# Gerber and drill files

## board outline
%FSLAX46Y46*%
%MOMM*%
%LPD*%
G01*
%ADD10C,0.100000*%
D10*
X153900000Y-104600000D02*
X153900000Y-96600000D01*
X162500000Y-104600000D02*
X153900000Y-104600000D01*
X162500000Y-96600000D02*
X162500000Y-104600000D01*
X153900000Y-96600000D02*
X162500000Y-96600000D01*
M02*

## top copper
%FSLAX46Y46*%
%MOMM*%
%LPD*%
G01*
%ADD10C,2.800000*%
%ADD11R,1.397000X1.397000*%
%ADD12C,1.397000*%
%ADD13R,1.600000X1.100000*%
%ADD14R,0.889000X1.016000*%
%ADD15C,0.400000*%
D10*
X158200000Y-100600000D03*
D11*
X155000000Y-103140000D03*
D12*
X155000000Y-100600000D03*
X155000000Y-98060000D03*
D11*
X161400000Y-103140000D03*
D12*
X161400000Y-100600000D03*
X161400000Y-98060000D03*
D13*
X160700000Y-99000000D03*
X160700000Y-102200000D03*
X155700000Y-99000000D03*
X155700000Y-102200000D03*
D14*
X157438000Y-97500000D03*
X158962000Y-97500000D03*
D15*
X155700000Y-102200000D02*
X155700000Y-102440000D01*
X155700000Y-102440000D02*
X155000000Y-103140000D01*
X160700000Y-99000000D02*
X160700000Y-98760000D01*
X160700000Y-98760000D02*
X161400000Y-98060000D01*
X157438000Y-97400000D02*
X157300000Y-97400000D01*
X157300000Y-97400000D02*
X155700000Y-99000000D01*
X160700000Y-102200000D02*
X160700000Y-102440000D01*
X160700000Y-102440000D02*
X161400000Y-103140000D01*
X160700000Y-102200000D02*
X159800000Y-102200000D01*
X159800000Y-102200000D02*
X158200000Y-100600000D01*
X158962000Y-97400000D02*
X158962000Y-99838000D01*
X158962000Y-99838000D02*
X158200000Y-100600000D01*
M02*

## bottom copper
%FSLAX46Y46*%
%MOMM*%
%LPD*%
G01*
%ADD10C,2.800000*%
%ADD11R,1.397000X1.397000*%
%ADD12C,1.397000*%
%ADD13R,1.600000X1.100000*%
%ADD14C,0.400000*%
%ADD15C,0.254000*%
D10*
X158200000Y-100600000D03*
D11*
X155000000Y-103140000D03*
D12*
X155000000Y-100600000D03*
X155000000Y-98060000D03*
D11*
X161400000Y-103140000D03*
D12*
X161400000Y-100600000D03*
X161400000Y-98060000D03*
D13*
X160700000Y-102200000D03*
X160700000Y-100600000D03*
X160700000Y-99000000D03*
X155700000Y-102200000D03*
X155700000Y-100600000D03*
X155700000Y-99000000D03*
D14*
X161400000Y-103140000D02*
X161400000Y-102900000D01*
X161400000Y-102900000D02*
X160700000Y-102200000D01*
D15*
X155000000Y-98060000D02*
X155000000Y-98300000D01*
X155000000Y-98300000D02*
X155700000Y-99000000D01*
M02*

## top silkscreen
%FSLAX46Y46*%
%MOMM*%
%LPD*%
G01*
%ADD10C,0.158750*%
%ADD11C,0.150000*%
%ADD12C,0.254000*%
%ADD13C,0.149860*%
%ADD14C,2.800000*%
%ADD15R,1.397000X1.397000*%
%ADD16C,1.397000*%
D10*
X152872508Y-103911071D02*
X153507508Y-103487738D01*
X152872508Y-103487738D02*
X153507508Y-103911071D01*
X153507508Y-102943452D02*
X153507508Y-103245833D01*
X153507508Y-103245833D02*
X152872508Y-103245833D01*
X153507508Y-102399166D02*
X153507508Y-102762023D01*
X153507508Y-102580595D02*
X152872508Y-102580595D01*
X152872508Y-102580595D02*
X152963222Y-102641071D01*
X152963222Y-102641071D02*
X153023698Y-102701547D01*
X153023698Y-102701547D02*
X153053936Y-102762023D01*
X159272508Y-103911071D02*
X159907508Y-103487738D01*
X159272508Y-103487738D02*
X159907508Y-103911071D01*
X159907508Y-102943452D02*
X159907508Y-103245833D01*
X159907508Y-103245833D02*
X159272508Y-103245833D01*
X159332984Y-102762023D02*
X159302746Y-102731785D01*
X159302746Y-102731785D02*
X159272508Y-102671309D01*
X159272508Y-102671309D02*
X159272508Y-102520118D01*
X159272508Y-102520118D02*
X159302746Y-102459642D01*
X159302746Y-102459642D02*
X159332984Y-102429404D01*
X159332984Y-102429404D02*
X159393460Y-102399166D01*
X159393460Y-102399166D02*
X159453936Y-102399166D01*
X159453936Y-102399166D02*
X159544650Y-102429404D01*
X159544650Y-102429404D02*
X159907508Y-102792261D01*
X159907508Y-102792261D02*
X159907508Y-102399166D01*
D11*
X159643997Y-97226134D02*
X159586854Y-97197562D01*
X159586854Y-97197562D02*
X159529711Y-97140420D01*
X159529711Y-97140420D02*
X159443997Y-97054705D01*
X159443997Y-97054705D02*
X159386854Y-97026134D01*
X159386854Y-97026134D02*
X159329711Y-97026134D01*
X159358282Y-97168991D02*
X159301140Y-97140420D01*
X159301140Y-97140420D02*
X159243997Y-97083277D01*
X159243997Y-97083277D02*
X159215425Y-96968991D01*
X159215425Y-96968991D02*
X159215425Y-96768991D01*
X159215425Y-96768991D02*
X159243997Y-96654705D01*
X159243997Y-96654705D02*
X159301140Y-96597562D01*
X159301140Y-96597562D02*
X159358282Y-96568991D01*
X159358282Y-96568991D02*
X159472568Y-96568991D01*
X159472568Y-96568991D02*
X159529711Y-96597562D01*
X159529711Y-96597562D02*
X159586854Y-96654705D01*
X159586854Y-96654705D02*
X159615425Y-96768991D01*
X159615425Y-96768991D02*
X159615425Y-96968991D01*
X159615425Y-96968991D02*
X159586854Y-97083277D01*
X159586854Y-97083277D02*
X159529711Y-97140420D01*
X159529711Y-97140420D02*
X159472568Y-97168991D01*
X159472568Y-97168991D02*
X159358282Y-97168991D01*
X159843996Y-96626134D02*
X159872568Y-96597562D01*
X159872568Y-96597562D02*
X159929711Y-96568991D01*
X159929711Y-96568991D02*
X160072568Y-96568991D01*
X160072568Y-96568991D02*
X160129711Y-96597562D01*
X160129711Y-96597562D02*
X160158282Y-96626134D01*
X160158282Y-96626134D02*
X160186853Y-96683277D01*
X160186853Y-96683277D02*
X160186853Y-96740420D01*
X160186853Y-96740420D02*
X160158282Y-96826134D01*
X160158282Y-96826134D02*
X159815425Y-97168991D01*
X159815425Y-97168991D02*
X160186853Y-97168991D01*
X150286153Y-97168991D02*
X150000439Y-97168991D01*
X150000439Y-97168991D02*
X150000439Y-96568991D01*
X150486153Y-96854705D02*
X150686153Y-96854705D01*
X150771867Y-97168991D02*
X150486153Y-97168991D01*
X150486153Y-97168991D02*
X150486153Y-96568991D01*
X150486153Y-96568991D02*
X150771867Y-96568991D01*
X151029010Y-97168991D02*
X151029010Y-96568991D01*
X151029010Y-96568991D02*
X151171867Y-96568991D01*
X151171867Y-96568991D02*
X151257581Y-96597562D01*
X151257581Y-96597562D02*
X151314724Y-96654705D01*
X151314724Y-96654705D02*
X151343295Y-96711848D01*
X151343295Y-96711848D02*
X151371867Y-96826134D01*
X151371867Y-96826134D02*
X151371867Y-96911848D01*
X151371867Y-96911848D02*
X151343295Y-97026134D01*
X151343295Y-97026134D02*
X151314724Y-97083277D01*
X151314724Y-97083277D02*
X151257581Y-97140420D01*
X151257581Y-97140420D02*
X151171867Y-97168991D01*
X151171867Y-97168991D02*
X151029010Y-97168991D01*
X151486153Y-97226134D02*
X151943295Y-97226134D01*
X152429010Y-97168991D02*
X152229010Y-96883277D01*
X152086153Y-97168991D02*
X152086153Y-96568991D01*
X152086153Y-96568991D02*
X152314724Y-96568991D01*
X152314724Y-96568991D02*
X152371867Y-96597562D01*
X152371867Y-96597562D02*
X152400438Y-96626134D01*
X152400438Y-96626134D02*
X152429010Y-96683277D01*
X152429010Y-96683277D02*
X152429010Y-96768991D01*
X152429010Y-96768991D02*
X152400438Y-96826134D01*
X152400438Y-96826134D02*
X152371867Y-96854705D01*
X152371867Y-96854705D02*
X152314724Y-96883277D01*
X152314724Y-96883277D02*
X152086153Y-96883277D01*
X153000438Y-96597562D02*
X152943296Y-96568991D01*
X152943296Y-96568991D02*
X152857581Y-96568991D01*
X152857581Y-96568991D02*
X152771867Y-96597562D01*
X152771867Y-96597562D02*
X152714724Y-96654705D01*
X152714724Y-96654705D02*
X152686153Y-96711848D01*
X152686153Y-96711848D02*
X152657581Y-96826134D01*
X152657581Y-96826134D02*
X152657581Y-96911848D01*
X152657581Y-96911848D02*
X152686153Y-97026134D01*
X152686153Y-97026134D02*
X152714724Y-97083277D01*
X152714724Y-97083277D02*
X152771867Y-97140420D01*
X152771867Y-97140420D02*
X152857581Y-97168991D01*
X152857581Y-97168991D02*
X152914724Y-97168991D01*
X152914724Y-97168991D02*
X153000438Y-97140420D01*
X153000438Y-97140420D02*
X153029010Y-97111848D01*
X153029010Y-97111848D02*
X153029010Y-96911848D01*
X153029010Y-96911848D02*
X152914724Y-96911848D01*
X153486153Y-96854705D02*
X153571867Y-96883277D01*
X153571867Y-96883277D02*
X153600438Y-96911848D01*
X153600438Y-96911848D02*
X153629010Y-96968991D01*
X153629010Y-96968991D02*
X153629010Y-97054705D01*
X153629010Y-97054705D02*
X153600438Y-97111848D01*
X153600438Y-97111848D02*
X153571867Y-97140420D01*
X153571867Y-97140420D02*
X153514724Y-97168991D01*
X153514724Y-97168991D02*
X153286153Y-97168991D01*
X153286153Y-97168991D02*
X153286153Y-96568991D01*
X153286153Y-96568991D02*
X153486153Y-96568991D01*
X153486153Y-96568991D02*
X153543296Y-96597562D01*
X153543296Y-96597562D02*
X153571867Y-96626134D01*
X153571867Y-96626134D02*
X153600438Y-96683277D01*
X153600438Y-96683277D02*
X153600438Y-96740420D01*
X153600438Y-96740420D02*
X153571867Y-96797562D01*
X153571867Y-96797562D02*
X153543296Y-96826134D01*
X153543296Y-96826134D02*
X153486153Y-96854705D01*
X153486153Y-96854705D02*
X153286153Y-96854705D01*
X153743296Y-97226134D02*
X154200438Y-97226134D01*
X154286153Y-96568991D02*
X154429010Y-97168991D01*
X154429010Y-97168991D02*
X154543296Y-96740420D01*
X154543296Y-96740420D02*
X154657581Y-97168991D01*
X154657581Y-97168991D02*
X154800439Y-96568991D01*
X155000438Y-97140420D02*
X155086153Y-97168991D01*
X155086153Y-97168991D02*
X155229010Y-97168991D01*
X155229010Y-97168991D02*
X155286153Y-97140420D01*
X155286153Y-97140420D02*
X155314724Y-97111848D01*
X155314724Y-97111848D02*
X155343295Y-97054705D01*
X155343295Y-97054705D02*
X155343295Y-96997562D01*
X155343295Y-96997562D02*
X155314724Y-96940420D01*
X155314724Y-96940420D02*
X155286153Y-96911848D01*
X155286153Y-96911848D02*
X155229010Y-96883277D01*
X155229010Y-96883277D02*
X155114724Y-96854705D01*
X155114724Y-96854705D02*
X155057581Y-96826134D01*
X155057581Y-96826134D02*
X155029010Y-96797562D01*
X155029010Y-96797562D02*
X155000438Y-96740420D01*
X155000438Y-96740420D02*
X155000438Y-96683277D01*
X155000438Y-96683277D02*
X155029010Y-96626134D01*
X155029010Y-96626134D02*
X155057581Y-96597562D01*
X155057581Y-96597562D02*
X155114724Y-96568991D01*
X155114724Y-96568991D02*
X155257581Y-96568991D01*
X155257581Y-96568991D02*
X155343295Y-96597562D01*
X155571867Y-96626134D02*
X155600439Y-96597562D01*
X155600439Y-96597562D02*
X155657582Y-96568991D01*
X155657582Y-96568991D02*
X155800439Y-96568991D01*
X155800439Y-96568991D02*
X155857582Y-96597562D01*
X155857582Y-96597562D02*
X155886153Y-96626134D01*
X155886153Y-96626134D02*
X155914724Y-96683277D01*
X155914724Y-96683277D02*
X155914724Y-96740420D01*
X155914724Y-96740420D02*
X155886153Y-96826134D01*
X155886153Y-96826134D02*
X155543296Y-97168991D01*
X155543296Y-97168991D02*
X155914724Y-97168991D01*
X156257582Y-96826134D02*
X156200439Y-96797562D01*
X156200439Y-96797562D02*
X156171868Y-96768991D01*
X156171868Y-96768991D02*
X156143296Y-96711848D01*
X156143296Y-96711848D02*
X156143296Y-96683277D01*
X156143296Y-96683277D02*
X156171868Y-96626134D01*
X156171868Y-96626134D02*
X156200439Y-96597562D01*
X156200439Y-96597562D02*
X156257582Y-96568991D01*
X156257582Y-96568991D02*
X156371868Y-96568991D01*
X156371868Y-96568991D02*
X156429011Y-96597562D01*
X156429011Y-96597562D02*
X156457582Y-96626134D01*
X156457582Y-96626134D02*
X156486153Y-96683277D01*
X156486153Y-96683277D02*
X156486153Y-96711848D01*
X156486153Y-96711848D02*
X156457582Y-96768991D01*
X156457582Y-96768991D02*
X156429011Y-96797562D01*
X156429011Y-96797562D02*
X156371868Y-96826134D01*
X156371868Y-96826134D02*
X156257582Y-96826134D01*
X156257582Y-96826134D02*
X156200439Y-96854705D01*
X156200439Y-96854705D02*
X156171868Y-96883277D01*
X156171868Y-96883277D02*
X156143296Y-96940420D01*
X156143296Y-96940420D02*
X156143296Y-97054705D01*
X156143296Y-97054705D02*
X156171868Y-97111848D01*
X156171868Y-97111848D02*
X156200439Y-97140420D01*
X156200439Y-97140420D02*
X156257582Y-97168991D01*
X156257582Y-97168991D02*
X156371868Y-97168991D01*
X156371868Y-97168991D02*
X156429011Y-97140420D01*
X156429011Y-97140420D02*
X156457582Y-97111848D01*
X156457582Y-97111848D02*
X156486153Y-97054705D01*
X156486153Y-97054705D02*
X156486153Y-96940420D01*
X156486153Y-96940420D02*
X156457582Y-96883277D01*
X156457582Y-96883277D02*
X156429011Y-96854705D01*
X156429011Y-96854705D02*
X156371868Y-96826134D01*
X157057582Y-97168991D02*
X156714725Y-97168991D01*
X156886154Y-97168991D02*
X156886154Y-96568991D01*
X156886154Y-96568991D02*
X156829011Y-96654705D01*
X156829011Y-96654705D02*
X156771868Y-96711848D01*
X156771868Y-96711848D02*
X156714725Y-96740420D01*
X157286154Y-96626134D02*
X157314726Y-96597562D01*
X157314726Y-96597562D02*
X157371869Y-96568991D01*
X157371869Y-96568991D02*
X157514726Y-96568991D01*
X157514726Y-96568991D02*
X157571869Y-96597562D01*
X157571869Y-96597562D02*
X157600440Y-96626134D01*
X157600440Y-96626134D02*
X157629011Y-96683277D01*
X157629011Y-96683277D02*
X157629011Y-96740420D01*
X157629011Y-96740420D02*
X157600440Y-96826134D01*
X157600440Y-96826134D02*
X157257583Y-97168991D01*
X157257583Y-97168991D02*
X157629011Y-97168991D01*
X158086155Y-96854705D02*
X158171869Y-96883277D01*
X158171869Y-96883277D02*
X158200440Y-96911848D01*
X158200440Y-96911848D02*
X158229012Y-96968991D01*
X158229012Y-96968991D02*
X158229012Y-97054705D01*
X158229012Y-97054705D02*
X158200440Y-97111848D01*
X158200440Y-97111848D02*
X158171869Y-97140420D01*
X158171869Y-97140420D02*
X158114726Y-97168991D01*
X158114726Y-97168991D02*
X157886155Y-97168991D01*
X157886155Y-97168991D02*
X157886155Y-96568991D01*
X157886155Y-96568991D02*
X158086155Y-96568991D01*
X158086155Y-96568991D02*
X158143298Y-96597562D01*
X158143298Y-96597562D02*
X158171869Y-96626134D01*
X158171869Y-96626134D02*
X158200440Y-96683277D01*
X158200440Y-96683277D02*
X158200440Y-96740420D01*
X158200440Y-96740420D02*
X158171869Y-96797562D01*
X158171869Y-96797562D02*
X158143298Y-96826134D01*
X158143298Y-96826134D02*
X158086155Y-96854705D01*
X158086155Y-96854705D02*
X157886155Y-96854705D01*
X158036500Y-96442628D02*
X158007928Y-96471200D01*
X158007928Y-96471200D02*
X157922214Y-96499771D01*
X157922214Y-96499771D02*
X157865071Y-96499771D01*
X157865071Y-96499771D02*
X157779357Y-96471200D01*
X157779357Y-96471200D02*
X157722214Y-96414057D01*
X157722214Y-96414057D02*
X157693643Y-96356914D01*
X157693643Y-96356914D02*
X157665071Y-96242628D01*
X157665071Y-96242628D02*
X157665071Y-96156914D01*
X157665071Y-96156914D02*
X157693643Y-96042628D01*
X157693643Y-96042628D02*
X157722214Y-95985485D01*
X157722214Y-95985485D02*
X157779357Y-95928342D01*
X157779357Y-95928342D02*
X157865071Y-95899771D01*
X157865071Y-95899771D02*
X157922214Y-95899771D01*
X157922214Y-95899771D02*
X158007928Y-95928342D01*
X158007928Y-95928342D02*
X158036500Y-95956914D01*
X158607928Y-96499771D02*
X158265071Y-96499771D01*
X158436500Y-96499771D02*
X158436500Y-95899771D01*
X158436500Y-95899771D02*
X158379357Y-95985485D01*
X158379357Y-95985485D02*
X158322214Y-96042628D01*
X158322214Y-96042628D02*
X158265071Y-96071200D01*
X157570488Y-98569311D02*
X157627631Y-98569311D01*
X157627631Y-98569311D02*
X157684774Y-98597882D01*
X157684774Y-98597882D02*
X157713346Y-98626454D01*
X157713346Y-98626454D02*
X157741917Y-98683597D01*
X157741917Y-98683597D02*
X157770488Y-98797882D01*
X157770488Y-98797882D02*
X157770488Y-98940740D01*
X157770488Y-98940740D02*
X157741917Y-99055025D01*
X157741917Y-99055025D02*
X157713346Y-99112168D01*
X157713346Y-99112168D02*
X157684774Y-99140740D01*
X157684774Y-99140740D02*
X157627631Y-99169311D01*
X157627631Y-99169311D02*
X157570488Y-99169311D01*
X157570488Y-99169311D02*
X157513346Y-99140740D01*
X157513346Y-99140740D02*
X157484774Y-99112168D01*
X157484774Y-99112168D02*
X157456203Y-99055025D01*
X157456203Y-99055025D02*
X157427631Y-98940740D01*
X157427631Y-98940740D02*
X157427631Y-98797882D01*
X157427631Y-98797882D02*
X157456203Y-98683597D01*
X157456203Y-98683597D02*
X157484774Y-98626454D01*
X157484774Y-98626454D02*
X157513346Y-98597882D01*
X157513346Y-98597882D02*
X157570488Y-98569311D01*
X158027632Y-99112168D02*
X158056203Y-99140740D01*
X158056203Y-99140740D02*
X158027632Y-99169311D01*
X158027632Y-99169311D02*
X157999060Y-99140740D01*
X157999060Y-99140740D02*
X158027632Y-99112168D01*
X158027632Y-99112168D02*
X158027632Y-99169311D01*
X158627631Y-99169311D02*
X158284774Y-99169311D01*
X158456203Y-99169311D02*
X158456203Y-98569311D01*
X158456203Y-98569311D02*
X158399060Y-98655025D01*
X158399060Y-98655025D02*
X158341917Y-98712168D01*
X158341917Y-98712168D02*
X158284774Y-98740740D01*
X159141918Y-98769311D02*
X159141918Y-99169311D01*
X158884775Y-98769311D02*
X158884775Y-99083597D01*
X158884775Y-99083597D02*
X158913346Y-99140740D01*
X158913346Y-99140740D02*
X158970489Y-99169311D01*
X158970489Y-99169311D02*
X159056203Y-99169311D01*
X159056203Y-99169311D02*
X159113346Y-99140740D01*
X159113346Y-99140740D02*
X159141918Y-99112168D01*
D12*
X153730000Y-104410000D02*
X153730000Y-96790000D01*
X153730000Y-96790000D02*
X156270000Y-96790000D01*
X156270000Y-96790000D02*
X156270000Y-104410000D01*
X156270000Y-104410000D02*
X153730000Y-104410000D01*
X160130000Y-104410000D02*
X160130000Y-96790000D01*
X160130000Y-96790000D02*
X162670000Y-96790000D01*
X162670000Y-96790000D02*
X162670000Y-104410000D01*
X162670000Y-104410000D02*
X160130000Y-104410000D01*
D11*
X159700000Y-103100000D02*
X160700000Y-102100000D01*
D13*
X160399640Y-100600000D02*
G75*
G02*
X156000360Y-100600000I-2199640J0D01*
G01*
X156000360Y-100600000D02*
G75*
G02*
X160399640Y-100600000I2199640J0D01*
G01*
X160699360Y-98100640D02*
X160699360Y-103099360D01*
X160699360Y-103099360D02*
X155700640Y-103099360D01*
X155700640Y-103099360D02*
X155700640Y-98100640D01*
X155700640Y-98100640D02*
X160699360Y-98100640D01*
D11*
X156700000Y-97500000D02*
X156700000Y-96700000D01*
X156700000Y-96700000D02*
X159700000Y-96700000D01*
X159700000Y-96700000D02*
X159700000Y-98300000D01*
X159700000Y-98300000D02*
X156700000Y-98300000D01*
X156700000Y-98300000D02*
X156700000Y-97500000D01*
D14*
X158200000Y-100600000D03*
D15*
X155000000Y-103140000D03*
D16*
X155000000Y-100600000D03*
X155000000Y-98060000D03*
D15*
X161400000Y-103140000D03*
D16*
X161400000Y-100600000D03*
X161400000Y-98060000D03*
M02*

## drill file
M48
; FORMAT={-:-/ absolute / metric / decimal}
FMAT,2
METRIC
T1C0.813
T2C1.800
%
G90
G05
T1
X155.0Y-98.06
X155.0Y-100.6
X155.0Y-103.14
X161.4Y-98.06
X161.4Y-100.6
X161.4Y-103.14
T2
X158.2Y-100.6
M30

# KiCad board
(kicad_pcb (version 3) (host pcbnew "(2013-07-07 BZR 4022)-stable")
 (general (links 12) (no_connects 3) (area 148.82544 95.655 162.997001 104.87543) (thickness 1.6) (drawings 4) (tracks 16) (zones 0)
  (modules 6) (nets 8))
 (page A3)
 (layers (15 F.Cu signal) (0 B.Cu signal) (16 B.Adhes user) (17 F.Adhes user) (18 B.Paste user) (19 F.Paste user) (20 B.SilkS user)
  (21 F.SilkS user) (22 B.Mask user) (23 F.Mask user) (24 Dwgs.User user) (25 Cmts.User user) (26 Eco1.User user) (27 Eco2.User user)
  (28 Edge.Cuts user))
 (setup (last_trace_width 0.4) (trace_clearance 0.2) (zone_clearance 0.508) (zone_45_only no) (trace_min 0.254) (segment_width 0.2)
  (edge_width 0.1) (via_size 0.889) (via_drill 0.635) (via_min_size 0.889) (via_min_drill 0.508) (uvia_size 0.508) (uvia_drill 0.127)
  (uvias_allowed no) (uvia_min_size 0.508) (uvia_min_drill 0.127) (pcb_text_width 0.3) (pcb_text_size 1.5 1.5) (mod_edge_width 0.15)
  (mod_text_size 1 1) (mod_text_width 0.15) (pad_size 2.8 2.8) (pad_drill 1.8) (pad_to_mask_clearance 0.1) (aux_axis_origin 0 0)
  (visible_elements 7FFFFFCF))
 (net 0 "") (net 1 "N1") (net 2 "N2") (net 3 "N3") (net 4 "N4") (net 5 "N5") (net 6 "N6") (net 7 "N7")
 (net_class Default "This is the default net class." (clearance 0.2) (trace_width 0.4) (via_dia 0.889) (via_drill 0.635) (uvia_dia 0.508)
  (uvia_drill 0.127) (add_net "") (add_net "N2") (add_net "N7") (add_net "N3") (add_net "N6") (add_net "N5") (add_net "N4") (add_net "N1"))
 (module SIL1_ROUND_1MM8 (layer F.Cu) (at 158.2 100.6)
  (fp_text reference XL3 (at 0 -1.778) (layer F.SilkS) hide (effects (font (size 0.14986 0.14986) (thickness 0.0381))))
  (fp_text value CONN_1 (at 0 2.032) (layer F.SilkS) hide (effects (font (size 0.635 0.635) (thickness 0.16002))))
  (pad 1 thru_hole circle (at 0 0) (size 2.8 2.8) (drill 1.8) (layers *.Cu *.Mask F.SilkS) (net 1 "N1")))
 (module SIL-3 (layer F.Cu) (at 155 100.6 90)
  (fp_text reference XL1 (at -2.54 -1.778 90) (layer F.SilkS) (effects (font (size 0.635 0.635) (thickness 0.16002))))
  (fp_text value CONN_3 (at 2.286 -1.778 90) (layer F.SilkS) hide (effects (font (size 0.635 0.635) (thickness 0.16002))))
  (fp_line (start -3.81 -1.27) (end 3.81 -1.27) (layer F.SilkS) (width 0.254))
  (fp_line (start 3.81 -1.27) (end 3.81 1.27) (layer F.SilkS) (width 0.254))
  (fp_line (start 3.81 1.27) (end -3.81 1.27) (layer F.SilkS) (width 0.254))
  (fp_line (start -3.81 1.27) (end -3.81 -1.27) (layer F.SilkS) (width 0.254))
  (pad 1 thru_hole rect (at -2.54 0 90) (size 1.397 1.397) (drill 0.8128) (layers *.Cu *.Mask F.SilkS) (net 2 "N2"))
  (pad 2 thru_hole circle (at 0 0 90) (size 1.397 1.397) (drill 0.8128) (layers *.Cu *.Mask F.SilkS) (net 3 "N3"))
  (pad 3 thru_hole circle (at 2.54 0 90) (size 1.397 1.397) (drill 0.8128) (layers *.Cu *.Mask F.SilkS) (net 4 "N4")))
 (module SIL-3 (layer F.Cu) (at 161.4 100.6 90)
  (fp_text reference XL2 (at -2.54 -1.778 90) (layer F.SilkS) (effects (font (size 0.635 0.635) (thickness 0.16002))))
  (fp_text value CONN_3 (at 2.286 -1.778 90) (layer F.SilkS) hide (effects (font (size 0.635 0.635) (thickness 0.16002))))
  (fp_line (start -3.81 -1.27) (end 3.81 -1.27) (layer F.SilkS) (width 0.254))
  (fp_line (start 3.81 -1.27) (end 3.81 1.27) (layer F.SilkS) (width 0.254))
  (fp_line (start 3.81 1.27) (end -3.81 1.27) (layer F.SilkS) (width 0.254))
  (fp_line (start -3.81 1.27) (end -3.81 -1.27) (layer F.SilkS) (width 0.254))
  (pad 1 thru_hole rect (at -2.54 0 90) (size 1.397 1.397) (drill 0.8128) (layers *.Cu *.Mask F.SilkS) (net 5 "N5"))
  (pad 2 thru_hole circle (at 0 0 90) (size 1.397 1.397) (drill 0.8128) (layers *.Cu *.Mask F.SilkS) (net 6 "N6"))
  (pad 3 thru_hole circle (at 2.54 0 90) (size 1.397 1.397) (drill 0.8128) (layers *.Cu *.Mask F.SilkS) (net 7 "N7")))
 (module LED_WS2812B (layer F.Cu) (at 158.2 100.6)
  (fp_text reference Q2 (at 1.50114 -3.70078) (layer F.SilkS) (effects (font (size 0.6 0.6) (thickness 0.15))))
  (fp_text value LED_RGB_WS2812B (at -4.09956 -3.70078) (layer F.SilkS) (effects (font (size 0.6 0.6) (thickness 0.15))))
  (fp_line (start 1.5 2.5) (end 2.5 1.5) (layer F.SilkS) (width 0.15))
  (fp_circle (center 0 0) (end 0 2.19964) (layer F.SilkS) (width 0.14986))
  (fp_line (start 2.49936 -2.49936) (end 2.49936 2.49936) (layer F.SilkS) (width 0.14986))
  (fp_line (start 2.49936 2.49936) (end -2.49936 2.49936) (layer F.SilkS) (width 0.14986))
  (fp_line (start -2.49936 2.49936) (end -2.49936 -2.49936) (layer F.SilkS) (width 0.14986))
  (fp_line (start -2.49936 -2.49936) (end 2.49936 -2.49936) (layer F.SilkS) (width 0.14986))
  (pad 4 smd rect (at 2.5 -1.6) (size 1.6 1.1) (layers F.Cu F.Paste F.Mask) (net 7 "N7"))
  (pad 3 smd rect (at 2.5 1.6) (size 1.6 1.1) (layers F.Cu F.Paste F.Mask) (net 1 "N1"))
  (pad 1 smd rect (at -2.5 -1.6) (size 1.6 1.1) (layers F.Cu F.Paste F.Mask) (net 4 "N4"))
  (pad 2 smd rect (at -2.5 1.6) (size 1.6 1.1) (layers F.Cu F.Paste F.Mask) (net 2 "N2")))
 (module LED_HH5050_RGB (layer B.Cu) (at 158.2 100.6)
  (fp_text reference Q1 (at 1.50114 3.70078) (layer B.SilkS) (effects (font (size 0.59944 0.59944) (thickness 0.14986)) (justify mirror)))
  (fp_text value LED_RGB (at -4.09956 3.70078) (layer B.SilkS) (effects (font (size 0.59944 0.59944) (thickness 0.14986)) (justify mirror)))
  (pad GC smd rect (at 2.5 1.6) (size 1.6 1.1) (layers B.Cu B.Paste B.Mask) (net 5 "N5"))
  (pad RC smd rect (at 2.5 0) (size 1.6 1.1) (layers B.Cu B.Paste B.Mask) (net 6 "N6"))
  (pad BC smd rect (at 2.5 -1.6) (size 1.6 1.1) (layers B.Cu B.Paste B.Mask) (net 7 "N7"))
  (pad GA smd rect (at -2.5 1.6) (size 1.6 1.1) (layers B.Cu B.Paste B.Mask) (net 2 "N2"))
  (pad RA smd rect (at -2.5 0) (size 1.6 1.1) (layers B.Cu B.Paste B.Mask) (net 3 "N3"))
  (pad BA smd rect (at -2.5 -1.6) (size 1.6 1.1) (layers B.Cu B.Paste B.Mask) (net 4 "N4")))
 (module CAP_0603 (layer F.Cu) (at 158.2 97.5)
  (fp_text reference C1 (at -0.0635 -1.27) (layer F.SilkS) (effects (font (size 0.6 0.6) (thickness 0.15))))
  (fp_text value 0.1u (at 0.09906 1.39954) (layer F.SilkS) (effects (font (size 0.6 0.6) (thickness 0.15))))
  (fp_line (start -1.5 0) (end -1.5 -0.8) (layer F.SilkS) (width 0.15))
  (fp_line (start -1.5 -0.8) (end 1.5 -0.8) (layer F.SilkS) (width 0.15))
  (fp_line (start 1.5 -0.8) (end 1.5 0.8) (layer F.SilkS) (width 0.15))
  (fp_line (start 1.5 0.8) (end -1.5 0.8) (layer F.SilkS) (width 0.15))
  (fp_line (start -1.5 0.8) (end -1.5 0) (layer F.SilkS) (width 0.15))
  (pad 1 smd rect (at -0.762 0) (size 0.889 1.016) (layers F.Cu F.Paste F.Mask) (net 4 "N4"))
  (pad 2 smd rect (at 0.762 0) (size 0.889 1.016) (layers F.Cu F.Paste F.Mask) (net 1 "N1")))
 (gr_line (start 153.9 104.6) (end 153.9 96.6) (angle 90) (layer Edge.Cuts) (width 0.1))
 (gr_line (start 162.5 104.6) (end 153.9 104.6) (angle 90) (layer Edge.Cuts) (width 0.1))
 (gr_line (start 162.5 96.6) (end 162.5 104.6) (angle 90) (layer Edge.Cuts) (width 0.1))
 (gr_line (start 153.9 96.6) (end 162.5 96.6) (angle 90) (layer Edge.Cuts) (width 0.1))
 (segment (start 155.7 102.2) (end 155.7 102.44) (width 0.4) (layer F.Cu) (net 2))
 (segment (start 155.7 102.44) (end 155 103.14) (width 0.4) (layer F.Cu) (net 2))
 (segment (start 160.7 99) (end 160.7 98.76) (width 0.4) (layer F.Cu) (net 7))
 (segment (start 160.7 98.76) (end 161.4 98.06) (width 0.4) (layer F.Cu) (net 7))
 (segment (start 161.4 103.14) (end 161.4 102.9) (width 0.4) (layer B.Cu) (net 5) (status C00000))
 (segment (start 161.4 102.9) (end 160.7 102.2) (width 0.4) (layer B.Cu) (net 5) (status C00000))
 (segment (start 157.438 97.4) (end 157.3 97.4) (width 0.4) (layer F.Cu) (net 4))
 (segment (start 157.3 97.4) (end 155.7 99) (width 0.4) (layer F.Cu) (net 4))
 (segment (start 155 98.06) (end 155 98.3) (width 0.254) (layer B.Cu) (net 4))
 (segment (start 155 98.3) (end 155.7 99) (width 0.254) (layer B.Cu) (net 4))
 (segment (start 160.7 102.2) (end 160.7 102.44) (width 0.4) (layer F.Cu) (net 1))
 (segment (start 160.7 102.44) (end 161.4 103.14) (width 0.4) (layer F.Cu) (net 1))
 (segment (start 160.7 102.2) (end 159.8 102.2) (width 0.4) (layer F.Cu) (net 1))
 (segment (start 159.8 102.2) (end 158.2 100.6) (width 0.4) (layer F.Cu) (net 1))
 (segment (start 158.962 97.4) (end 158.962 99.838) (width 0.4) (layer F.Cu) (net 1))
 (segment (start 158.962 99.838) (end 158.2 100.6) (width 0.4) (layer F.Cu) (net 1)))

